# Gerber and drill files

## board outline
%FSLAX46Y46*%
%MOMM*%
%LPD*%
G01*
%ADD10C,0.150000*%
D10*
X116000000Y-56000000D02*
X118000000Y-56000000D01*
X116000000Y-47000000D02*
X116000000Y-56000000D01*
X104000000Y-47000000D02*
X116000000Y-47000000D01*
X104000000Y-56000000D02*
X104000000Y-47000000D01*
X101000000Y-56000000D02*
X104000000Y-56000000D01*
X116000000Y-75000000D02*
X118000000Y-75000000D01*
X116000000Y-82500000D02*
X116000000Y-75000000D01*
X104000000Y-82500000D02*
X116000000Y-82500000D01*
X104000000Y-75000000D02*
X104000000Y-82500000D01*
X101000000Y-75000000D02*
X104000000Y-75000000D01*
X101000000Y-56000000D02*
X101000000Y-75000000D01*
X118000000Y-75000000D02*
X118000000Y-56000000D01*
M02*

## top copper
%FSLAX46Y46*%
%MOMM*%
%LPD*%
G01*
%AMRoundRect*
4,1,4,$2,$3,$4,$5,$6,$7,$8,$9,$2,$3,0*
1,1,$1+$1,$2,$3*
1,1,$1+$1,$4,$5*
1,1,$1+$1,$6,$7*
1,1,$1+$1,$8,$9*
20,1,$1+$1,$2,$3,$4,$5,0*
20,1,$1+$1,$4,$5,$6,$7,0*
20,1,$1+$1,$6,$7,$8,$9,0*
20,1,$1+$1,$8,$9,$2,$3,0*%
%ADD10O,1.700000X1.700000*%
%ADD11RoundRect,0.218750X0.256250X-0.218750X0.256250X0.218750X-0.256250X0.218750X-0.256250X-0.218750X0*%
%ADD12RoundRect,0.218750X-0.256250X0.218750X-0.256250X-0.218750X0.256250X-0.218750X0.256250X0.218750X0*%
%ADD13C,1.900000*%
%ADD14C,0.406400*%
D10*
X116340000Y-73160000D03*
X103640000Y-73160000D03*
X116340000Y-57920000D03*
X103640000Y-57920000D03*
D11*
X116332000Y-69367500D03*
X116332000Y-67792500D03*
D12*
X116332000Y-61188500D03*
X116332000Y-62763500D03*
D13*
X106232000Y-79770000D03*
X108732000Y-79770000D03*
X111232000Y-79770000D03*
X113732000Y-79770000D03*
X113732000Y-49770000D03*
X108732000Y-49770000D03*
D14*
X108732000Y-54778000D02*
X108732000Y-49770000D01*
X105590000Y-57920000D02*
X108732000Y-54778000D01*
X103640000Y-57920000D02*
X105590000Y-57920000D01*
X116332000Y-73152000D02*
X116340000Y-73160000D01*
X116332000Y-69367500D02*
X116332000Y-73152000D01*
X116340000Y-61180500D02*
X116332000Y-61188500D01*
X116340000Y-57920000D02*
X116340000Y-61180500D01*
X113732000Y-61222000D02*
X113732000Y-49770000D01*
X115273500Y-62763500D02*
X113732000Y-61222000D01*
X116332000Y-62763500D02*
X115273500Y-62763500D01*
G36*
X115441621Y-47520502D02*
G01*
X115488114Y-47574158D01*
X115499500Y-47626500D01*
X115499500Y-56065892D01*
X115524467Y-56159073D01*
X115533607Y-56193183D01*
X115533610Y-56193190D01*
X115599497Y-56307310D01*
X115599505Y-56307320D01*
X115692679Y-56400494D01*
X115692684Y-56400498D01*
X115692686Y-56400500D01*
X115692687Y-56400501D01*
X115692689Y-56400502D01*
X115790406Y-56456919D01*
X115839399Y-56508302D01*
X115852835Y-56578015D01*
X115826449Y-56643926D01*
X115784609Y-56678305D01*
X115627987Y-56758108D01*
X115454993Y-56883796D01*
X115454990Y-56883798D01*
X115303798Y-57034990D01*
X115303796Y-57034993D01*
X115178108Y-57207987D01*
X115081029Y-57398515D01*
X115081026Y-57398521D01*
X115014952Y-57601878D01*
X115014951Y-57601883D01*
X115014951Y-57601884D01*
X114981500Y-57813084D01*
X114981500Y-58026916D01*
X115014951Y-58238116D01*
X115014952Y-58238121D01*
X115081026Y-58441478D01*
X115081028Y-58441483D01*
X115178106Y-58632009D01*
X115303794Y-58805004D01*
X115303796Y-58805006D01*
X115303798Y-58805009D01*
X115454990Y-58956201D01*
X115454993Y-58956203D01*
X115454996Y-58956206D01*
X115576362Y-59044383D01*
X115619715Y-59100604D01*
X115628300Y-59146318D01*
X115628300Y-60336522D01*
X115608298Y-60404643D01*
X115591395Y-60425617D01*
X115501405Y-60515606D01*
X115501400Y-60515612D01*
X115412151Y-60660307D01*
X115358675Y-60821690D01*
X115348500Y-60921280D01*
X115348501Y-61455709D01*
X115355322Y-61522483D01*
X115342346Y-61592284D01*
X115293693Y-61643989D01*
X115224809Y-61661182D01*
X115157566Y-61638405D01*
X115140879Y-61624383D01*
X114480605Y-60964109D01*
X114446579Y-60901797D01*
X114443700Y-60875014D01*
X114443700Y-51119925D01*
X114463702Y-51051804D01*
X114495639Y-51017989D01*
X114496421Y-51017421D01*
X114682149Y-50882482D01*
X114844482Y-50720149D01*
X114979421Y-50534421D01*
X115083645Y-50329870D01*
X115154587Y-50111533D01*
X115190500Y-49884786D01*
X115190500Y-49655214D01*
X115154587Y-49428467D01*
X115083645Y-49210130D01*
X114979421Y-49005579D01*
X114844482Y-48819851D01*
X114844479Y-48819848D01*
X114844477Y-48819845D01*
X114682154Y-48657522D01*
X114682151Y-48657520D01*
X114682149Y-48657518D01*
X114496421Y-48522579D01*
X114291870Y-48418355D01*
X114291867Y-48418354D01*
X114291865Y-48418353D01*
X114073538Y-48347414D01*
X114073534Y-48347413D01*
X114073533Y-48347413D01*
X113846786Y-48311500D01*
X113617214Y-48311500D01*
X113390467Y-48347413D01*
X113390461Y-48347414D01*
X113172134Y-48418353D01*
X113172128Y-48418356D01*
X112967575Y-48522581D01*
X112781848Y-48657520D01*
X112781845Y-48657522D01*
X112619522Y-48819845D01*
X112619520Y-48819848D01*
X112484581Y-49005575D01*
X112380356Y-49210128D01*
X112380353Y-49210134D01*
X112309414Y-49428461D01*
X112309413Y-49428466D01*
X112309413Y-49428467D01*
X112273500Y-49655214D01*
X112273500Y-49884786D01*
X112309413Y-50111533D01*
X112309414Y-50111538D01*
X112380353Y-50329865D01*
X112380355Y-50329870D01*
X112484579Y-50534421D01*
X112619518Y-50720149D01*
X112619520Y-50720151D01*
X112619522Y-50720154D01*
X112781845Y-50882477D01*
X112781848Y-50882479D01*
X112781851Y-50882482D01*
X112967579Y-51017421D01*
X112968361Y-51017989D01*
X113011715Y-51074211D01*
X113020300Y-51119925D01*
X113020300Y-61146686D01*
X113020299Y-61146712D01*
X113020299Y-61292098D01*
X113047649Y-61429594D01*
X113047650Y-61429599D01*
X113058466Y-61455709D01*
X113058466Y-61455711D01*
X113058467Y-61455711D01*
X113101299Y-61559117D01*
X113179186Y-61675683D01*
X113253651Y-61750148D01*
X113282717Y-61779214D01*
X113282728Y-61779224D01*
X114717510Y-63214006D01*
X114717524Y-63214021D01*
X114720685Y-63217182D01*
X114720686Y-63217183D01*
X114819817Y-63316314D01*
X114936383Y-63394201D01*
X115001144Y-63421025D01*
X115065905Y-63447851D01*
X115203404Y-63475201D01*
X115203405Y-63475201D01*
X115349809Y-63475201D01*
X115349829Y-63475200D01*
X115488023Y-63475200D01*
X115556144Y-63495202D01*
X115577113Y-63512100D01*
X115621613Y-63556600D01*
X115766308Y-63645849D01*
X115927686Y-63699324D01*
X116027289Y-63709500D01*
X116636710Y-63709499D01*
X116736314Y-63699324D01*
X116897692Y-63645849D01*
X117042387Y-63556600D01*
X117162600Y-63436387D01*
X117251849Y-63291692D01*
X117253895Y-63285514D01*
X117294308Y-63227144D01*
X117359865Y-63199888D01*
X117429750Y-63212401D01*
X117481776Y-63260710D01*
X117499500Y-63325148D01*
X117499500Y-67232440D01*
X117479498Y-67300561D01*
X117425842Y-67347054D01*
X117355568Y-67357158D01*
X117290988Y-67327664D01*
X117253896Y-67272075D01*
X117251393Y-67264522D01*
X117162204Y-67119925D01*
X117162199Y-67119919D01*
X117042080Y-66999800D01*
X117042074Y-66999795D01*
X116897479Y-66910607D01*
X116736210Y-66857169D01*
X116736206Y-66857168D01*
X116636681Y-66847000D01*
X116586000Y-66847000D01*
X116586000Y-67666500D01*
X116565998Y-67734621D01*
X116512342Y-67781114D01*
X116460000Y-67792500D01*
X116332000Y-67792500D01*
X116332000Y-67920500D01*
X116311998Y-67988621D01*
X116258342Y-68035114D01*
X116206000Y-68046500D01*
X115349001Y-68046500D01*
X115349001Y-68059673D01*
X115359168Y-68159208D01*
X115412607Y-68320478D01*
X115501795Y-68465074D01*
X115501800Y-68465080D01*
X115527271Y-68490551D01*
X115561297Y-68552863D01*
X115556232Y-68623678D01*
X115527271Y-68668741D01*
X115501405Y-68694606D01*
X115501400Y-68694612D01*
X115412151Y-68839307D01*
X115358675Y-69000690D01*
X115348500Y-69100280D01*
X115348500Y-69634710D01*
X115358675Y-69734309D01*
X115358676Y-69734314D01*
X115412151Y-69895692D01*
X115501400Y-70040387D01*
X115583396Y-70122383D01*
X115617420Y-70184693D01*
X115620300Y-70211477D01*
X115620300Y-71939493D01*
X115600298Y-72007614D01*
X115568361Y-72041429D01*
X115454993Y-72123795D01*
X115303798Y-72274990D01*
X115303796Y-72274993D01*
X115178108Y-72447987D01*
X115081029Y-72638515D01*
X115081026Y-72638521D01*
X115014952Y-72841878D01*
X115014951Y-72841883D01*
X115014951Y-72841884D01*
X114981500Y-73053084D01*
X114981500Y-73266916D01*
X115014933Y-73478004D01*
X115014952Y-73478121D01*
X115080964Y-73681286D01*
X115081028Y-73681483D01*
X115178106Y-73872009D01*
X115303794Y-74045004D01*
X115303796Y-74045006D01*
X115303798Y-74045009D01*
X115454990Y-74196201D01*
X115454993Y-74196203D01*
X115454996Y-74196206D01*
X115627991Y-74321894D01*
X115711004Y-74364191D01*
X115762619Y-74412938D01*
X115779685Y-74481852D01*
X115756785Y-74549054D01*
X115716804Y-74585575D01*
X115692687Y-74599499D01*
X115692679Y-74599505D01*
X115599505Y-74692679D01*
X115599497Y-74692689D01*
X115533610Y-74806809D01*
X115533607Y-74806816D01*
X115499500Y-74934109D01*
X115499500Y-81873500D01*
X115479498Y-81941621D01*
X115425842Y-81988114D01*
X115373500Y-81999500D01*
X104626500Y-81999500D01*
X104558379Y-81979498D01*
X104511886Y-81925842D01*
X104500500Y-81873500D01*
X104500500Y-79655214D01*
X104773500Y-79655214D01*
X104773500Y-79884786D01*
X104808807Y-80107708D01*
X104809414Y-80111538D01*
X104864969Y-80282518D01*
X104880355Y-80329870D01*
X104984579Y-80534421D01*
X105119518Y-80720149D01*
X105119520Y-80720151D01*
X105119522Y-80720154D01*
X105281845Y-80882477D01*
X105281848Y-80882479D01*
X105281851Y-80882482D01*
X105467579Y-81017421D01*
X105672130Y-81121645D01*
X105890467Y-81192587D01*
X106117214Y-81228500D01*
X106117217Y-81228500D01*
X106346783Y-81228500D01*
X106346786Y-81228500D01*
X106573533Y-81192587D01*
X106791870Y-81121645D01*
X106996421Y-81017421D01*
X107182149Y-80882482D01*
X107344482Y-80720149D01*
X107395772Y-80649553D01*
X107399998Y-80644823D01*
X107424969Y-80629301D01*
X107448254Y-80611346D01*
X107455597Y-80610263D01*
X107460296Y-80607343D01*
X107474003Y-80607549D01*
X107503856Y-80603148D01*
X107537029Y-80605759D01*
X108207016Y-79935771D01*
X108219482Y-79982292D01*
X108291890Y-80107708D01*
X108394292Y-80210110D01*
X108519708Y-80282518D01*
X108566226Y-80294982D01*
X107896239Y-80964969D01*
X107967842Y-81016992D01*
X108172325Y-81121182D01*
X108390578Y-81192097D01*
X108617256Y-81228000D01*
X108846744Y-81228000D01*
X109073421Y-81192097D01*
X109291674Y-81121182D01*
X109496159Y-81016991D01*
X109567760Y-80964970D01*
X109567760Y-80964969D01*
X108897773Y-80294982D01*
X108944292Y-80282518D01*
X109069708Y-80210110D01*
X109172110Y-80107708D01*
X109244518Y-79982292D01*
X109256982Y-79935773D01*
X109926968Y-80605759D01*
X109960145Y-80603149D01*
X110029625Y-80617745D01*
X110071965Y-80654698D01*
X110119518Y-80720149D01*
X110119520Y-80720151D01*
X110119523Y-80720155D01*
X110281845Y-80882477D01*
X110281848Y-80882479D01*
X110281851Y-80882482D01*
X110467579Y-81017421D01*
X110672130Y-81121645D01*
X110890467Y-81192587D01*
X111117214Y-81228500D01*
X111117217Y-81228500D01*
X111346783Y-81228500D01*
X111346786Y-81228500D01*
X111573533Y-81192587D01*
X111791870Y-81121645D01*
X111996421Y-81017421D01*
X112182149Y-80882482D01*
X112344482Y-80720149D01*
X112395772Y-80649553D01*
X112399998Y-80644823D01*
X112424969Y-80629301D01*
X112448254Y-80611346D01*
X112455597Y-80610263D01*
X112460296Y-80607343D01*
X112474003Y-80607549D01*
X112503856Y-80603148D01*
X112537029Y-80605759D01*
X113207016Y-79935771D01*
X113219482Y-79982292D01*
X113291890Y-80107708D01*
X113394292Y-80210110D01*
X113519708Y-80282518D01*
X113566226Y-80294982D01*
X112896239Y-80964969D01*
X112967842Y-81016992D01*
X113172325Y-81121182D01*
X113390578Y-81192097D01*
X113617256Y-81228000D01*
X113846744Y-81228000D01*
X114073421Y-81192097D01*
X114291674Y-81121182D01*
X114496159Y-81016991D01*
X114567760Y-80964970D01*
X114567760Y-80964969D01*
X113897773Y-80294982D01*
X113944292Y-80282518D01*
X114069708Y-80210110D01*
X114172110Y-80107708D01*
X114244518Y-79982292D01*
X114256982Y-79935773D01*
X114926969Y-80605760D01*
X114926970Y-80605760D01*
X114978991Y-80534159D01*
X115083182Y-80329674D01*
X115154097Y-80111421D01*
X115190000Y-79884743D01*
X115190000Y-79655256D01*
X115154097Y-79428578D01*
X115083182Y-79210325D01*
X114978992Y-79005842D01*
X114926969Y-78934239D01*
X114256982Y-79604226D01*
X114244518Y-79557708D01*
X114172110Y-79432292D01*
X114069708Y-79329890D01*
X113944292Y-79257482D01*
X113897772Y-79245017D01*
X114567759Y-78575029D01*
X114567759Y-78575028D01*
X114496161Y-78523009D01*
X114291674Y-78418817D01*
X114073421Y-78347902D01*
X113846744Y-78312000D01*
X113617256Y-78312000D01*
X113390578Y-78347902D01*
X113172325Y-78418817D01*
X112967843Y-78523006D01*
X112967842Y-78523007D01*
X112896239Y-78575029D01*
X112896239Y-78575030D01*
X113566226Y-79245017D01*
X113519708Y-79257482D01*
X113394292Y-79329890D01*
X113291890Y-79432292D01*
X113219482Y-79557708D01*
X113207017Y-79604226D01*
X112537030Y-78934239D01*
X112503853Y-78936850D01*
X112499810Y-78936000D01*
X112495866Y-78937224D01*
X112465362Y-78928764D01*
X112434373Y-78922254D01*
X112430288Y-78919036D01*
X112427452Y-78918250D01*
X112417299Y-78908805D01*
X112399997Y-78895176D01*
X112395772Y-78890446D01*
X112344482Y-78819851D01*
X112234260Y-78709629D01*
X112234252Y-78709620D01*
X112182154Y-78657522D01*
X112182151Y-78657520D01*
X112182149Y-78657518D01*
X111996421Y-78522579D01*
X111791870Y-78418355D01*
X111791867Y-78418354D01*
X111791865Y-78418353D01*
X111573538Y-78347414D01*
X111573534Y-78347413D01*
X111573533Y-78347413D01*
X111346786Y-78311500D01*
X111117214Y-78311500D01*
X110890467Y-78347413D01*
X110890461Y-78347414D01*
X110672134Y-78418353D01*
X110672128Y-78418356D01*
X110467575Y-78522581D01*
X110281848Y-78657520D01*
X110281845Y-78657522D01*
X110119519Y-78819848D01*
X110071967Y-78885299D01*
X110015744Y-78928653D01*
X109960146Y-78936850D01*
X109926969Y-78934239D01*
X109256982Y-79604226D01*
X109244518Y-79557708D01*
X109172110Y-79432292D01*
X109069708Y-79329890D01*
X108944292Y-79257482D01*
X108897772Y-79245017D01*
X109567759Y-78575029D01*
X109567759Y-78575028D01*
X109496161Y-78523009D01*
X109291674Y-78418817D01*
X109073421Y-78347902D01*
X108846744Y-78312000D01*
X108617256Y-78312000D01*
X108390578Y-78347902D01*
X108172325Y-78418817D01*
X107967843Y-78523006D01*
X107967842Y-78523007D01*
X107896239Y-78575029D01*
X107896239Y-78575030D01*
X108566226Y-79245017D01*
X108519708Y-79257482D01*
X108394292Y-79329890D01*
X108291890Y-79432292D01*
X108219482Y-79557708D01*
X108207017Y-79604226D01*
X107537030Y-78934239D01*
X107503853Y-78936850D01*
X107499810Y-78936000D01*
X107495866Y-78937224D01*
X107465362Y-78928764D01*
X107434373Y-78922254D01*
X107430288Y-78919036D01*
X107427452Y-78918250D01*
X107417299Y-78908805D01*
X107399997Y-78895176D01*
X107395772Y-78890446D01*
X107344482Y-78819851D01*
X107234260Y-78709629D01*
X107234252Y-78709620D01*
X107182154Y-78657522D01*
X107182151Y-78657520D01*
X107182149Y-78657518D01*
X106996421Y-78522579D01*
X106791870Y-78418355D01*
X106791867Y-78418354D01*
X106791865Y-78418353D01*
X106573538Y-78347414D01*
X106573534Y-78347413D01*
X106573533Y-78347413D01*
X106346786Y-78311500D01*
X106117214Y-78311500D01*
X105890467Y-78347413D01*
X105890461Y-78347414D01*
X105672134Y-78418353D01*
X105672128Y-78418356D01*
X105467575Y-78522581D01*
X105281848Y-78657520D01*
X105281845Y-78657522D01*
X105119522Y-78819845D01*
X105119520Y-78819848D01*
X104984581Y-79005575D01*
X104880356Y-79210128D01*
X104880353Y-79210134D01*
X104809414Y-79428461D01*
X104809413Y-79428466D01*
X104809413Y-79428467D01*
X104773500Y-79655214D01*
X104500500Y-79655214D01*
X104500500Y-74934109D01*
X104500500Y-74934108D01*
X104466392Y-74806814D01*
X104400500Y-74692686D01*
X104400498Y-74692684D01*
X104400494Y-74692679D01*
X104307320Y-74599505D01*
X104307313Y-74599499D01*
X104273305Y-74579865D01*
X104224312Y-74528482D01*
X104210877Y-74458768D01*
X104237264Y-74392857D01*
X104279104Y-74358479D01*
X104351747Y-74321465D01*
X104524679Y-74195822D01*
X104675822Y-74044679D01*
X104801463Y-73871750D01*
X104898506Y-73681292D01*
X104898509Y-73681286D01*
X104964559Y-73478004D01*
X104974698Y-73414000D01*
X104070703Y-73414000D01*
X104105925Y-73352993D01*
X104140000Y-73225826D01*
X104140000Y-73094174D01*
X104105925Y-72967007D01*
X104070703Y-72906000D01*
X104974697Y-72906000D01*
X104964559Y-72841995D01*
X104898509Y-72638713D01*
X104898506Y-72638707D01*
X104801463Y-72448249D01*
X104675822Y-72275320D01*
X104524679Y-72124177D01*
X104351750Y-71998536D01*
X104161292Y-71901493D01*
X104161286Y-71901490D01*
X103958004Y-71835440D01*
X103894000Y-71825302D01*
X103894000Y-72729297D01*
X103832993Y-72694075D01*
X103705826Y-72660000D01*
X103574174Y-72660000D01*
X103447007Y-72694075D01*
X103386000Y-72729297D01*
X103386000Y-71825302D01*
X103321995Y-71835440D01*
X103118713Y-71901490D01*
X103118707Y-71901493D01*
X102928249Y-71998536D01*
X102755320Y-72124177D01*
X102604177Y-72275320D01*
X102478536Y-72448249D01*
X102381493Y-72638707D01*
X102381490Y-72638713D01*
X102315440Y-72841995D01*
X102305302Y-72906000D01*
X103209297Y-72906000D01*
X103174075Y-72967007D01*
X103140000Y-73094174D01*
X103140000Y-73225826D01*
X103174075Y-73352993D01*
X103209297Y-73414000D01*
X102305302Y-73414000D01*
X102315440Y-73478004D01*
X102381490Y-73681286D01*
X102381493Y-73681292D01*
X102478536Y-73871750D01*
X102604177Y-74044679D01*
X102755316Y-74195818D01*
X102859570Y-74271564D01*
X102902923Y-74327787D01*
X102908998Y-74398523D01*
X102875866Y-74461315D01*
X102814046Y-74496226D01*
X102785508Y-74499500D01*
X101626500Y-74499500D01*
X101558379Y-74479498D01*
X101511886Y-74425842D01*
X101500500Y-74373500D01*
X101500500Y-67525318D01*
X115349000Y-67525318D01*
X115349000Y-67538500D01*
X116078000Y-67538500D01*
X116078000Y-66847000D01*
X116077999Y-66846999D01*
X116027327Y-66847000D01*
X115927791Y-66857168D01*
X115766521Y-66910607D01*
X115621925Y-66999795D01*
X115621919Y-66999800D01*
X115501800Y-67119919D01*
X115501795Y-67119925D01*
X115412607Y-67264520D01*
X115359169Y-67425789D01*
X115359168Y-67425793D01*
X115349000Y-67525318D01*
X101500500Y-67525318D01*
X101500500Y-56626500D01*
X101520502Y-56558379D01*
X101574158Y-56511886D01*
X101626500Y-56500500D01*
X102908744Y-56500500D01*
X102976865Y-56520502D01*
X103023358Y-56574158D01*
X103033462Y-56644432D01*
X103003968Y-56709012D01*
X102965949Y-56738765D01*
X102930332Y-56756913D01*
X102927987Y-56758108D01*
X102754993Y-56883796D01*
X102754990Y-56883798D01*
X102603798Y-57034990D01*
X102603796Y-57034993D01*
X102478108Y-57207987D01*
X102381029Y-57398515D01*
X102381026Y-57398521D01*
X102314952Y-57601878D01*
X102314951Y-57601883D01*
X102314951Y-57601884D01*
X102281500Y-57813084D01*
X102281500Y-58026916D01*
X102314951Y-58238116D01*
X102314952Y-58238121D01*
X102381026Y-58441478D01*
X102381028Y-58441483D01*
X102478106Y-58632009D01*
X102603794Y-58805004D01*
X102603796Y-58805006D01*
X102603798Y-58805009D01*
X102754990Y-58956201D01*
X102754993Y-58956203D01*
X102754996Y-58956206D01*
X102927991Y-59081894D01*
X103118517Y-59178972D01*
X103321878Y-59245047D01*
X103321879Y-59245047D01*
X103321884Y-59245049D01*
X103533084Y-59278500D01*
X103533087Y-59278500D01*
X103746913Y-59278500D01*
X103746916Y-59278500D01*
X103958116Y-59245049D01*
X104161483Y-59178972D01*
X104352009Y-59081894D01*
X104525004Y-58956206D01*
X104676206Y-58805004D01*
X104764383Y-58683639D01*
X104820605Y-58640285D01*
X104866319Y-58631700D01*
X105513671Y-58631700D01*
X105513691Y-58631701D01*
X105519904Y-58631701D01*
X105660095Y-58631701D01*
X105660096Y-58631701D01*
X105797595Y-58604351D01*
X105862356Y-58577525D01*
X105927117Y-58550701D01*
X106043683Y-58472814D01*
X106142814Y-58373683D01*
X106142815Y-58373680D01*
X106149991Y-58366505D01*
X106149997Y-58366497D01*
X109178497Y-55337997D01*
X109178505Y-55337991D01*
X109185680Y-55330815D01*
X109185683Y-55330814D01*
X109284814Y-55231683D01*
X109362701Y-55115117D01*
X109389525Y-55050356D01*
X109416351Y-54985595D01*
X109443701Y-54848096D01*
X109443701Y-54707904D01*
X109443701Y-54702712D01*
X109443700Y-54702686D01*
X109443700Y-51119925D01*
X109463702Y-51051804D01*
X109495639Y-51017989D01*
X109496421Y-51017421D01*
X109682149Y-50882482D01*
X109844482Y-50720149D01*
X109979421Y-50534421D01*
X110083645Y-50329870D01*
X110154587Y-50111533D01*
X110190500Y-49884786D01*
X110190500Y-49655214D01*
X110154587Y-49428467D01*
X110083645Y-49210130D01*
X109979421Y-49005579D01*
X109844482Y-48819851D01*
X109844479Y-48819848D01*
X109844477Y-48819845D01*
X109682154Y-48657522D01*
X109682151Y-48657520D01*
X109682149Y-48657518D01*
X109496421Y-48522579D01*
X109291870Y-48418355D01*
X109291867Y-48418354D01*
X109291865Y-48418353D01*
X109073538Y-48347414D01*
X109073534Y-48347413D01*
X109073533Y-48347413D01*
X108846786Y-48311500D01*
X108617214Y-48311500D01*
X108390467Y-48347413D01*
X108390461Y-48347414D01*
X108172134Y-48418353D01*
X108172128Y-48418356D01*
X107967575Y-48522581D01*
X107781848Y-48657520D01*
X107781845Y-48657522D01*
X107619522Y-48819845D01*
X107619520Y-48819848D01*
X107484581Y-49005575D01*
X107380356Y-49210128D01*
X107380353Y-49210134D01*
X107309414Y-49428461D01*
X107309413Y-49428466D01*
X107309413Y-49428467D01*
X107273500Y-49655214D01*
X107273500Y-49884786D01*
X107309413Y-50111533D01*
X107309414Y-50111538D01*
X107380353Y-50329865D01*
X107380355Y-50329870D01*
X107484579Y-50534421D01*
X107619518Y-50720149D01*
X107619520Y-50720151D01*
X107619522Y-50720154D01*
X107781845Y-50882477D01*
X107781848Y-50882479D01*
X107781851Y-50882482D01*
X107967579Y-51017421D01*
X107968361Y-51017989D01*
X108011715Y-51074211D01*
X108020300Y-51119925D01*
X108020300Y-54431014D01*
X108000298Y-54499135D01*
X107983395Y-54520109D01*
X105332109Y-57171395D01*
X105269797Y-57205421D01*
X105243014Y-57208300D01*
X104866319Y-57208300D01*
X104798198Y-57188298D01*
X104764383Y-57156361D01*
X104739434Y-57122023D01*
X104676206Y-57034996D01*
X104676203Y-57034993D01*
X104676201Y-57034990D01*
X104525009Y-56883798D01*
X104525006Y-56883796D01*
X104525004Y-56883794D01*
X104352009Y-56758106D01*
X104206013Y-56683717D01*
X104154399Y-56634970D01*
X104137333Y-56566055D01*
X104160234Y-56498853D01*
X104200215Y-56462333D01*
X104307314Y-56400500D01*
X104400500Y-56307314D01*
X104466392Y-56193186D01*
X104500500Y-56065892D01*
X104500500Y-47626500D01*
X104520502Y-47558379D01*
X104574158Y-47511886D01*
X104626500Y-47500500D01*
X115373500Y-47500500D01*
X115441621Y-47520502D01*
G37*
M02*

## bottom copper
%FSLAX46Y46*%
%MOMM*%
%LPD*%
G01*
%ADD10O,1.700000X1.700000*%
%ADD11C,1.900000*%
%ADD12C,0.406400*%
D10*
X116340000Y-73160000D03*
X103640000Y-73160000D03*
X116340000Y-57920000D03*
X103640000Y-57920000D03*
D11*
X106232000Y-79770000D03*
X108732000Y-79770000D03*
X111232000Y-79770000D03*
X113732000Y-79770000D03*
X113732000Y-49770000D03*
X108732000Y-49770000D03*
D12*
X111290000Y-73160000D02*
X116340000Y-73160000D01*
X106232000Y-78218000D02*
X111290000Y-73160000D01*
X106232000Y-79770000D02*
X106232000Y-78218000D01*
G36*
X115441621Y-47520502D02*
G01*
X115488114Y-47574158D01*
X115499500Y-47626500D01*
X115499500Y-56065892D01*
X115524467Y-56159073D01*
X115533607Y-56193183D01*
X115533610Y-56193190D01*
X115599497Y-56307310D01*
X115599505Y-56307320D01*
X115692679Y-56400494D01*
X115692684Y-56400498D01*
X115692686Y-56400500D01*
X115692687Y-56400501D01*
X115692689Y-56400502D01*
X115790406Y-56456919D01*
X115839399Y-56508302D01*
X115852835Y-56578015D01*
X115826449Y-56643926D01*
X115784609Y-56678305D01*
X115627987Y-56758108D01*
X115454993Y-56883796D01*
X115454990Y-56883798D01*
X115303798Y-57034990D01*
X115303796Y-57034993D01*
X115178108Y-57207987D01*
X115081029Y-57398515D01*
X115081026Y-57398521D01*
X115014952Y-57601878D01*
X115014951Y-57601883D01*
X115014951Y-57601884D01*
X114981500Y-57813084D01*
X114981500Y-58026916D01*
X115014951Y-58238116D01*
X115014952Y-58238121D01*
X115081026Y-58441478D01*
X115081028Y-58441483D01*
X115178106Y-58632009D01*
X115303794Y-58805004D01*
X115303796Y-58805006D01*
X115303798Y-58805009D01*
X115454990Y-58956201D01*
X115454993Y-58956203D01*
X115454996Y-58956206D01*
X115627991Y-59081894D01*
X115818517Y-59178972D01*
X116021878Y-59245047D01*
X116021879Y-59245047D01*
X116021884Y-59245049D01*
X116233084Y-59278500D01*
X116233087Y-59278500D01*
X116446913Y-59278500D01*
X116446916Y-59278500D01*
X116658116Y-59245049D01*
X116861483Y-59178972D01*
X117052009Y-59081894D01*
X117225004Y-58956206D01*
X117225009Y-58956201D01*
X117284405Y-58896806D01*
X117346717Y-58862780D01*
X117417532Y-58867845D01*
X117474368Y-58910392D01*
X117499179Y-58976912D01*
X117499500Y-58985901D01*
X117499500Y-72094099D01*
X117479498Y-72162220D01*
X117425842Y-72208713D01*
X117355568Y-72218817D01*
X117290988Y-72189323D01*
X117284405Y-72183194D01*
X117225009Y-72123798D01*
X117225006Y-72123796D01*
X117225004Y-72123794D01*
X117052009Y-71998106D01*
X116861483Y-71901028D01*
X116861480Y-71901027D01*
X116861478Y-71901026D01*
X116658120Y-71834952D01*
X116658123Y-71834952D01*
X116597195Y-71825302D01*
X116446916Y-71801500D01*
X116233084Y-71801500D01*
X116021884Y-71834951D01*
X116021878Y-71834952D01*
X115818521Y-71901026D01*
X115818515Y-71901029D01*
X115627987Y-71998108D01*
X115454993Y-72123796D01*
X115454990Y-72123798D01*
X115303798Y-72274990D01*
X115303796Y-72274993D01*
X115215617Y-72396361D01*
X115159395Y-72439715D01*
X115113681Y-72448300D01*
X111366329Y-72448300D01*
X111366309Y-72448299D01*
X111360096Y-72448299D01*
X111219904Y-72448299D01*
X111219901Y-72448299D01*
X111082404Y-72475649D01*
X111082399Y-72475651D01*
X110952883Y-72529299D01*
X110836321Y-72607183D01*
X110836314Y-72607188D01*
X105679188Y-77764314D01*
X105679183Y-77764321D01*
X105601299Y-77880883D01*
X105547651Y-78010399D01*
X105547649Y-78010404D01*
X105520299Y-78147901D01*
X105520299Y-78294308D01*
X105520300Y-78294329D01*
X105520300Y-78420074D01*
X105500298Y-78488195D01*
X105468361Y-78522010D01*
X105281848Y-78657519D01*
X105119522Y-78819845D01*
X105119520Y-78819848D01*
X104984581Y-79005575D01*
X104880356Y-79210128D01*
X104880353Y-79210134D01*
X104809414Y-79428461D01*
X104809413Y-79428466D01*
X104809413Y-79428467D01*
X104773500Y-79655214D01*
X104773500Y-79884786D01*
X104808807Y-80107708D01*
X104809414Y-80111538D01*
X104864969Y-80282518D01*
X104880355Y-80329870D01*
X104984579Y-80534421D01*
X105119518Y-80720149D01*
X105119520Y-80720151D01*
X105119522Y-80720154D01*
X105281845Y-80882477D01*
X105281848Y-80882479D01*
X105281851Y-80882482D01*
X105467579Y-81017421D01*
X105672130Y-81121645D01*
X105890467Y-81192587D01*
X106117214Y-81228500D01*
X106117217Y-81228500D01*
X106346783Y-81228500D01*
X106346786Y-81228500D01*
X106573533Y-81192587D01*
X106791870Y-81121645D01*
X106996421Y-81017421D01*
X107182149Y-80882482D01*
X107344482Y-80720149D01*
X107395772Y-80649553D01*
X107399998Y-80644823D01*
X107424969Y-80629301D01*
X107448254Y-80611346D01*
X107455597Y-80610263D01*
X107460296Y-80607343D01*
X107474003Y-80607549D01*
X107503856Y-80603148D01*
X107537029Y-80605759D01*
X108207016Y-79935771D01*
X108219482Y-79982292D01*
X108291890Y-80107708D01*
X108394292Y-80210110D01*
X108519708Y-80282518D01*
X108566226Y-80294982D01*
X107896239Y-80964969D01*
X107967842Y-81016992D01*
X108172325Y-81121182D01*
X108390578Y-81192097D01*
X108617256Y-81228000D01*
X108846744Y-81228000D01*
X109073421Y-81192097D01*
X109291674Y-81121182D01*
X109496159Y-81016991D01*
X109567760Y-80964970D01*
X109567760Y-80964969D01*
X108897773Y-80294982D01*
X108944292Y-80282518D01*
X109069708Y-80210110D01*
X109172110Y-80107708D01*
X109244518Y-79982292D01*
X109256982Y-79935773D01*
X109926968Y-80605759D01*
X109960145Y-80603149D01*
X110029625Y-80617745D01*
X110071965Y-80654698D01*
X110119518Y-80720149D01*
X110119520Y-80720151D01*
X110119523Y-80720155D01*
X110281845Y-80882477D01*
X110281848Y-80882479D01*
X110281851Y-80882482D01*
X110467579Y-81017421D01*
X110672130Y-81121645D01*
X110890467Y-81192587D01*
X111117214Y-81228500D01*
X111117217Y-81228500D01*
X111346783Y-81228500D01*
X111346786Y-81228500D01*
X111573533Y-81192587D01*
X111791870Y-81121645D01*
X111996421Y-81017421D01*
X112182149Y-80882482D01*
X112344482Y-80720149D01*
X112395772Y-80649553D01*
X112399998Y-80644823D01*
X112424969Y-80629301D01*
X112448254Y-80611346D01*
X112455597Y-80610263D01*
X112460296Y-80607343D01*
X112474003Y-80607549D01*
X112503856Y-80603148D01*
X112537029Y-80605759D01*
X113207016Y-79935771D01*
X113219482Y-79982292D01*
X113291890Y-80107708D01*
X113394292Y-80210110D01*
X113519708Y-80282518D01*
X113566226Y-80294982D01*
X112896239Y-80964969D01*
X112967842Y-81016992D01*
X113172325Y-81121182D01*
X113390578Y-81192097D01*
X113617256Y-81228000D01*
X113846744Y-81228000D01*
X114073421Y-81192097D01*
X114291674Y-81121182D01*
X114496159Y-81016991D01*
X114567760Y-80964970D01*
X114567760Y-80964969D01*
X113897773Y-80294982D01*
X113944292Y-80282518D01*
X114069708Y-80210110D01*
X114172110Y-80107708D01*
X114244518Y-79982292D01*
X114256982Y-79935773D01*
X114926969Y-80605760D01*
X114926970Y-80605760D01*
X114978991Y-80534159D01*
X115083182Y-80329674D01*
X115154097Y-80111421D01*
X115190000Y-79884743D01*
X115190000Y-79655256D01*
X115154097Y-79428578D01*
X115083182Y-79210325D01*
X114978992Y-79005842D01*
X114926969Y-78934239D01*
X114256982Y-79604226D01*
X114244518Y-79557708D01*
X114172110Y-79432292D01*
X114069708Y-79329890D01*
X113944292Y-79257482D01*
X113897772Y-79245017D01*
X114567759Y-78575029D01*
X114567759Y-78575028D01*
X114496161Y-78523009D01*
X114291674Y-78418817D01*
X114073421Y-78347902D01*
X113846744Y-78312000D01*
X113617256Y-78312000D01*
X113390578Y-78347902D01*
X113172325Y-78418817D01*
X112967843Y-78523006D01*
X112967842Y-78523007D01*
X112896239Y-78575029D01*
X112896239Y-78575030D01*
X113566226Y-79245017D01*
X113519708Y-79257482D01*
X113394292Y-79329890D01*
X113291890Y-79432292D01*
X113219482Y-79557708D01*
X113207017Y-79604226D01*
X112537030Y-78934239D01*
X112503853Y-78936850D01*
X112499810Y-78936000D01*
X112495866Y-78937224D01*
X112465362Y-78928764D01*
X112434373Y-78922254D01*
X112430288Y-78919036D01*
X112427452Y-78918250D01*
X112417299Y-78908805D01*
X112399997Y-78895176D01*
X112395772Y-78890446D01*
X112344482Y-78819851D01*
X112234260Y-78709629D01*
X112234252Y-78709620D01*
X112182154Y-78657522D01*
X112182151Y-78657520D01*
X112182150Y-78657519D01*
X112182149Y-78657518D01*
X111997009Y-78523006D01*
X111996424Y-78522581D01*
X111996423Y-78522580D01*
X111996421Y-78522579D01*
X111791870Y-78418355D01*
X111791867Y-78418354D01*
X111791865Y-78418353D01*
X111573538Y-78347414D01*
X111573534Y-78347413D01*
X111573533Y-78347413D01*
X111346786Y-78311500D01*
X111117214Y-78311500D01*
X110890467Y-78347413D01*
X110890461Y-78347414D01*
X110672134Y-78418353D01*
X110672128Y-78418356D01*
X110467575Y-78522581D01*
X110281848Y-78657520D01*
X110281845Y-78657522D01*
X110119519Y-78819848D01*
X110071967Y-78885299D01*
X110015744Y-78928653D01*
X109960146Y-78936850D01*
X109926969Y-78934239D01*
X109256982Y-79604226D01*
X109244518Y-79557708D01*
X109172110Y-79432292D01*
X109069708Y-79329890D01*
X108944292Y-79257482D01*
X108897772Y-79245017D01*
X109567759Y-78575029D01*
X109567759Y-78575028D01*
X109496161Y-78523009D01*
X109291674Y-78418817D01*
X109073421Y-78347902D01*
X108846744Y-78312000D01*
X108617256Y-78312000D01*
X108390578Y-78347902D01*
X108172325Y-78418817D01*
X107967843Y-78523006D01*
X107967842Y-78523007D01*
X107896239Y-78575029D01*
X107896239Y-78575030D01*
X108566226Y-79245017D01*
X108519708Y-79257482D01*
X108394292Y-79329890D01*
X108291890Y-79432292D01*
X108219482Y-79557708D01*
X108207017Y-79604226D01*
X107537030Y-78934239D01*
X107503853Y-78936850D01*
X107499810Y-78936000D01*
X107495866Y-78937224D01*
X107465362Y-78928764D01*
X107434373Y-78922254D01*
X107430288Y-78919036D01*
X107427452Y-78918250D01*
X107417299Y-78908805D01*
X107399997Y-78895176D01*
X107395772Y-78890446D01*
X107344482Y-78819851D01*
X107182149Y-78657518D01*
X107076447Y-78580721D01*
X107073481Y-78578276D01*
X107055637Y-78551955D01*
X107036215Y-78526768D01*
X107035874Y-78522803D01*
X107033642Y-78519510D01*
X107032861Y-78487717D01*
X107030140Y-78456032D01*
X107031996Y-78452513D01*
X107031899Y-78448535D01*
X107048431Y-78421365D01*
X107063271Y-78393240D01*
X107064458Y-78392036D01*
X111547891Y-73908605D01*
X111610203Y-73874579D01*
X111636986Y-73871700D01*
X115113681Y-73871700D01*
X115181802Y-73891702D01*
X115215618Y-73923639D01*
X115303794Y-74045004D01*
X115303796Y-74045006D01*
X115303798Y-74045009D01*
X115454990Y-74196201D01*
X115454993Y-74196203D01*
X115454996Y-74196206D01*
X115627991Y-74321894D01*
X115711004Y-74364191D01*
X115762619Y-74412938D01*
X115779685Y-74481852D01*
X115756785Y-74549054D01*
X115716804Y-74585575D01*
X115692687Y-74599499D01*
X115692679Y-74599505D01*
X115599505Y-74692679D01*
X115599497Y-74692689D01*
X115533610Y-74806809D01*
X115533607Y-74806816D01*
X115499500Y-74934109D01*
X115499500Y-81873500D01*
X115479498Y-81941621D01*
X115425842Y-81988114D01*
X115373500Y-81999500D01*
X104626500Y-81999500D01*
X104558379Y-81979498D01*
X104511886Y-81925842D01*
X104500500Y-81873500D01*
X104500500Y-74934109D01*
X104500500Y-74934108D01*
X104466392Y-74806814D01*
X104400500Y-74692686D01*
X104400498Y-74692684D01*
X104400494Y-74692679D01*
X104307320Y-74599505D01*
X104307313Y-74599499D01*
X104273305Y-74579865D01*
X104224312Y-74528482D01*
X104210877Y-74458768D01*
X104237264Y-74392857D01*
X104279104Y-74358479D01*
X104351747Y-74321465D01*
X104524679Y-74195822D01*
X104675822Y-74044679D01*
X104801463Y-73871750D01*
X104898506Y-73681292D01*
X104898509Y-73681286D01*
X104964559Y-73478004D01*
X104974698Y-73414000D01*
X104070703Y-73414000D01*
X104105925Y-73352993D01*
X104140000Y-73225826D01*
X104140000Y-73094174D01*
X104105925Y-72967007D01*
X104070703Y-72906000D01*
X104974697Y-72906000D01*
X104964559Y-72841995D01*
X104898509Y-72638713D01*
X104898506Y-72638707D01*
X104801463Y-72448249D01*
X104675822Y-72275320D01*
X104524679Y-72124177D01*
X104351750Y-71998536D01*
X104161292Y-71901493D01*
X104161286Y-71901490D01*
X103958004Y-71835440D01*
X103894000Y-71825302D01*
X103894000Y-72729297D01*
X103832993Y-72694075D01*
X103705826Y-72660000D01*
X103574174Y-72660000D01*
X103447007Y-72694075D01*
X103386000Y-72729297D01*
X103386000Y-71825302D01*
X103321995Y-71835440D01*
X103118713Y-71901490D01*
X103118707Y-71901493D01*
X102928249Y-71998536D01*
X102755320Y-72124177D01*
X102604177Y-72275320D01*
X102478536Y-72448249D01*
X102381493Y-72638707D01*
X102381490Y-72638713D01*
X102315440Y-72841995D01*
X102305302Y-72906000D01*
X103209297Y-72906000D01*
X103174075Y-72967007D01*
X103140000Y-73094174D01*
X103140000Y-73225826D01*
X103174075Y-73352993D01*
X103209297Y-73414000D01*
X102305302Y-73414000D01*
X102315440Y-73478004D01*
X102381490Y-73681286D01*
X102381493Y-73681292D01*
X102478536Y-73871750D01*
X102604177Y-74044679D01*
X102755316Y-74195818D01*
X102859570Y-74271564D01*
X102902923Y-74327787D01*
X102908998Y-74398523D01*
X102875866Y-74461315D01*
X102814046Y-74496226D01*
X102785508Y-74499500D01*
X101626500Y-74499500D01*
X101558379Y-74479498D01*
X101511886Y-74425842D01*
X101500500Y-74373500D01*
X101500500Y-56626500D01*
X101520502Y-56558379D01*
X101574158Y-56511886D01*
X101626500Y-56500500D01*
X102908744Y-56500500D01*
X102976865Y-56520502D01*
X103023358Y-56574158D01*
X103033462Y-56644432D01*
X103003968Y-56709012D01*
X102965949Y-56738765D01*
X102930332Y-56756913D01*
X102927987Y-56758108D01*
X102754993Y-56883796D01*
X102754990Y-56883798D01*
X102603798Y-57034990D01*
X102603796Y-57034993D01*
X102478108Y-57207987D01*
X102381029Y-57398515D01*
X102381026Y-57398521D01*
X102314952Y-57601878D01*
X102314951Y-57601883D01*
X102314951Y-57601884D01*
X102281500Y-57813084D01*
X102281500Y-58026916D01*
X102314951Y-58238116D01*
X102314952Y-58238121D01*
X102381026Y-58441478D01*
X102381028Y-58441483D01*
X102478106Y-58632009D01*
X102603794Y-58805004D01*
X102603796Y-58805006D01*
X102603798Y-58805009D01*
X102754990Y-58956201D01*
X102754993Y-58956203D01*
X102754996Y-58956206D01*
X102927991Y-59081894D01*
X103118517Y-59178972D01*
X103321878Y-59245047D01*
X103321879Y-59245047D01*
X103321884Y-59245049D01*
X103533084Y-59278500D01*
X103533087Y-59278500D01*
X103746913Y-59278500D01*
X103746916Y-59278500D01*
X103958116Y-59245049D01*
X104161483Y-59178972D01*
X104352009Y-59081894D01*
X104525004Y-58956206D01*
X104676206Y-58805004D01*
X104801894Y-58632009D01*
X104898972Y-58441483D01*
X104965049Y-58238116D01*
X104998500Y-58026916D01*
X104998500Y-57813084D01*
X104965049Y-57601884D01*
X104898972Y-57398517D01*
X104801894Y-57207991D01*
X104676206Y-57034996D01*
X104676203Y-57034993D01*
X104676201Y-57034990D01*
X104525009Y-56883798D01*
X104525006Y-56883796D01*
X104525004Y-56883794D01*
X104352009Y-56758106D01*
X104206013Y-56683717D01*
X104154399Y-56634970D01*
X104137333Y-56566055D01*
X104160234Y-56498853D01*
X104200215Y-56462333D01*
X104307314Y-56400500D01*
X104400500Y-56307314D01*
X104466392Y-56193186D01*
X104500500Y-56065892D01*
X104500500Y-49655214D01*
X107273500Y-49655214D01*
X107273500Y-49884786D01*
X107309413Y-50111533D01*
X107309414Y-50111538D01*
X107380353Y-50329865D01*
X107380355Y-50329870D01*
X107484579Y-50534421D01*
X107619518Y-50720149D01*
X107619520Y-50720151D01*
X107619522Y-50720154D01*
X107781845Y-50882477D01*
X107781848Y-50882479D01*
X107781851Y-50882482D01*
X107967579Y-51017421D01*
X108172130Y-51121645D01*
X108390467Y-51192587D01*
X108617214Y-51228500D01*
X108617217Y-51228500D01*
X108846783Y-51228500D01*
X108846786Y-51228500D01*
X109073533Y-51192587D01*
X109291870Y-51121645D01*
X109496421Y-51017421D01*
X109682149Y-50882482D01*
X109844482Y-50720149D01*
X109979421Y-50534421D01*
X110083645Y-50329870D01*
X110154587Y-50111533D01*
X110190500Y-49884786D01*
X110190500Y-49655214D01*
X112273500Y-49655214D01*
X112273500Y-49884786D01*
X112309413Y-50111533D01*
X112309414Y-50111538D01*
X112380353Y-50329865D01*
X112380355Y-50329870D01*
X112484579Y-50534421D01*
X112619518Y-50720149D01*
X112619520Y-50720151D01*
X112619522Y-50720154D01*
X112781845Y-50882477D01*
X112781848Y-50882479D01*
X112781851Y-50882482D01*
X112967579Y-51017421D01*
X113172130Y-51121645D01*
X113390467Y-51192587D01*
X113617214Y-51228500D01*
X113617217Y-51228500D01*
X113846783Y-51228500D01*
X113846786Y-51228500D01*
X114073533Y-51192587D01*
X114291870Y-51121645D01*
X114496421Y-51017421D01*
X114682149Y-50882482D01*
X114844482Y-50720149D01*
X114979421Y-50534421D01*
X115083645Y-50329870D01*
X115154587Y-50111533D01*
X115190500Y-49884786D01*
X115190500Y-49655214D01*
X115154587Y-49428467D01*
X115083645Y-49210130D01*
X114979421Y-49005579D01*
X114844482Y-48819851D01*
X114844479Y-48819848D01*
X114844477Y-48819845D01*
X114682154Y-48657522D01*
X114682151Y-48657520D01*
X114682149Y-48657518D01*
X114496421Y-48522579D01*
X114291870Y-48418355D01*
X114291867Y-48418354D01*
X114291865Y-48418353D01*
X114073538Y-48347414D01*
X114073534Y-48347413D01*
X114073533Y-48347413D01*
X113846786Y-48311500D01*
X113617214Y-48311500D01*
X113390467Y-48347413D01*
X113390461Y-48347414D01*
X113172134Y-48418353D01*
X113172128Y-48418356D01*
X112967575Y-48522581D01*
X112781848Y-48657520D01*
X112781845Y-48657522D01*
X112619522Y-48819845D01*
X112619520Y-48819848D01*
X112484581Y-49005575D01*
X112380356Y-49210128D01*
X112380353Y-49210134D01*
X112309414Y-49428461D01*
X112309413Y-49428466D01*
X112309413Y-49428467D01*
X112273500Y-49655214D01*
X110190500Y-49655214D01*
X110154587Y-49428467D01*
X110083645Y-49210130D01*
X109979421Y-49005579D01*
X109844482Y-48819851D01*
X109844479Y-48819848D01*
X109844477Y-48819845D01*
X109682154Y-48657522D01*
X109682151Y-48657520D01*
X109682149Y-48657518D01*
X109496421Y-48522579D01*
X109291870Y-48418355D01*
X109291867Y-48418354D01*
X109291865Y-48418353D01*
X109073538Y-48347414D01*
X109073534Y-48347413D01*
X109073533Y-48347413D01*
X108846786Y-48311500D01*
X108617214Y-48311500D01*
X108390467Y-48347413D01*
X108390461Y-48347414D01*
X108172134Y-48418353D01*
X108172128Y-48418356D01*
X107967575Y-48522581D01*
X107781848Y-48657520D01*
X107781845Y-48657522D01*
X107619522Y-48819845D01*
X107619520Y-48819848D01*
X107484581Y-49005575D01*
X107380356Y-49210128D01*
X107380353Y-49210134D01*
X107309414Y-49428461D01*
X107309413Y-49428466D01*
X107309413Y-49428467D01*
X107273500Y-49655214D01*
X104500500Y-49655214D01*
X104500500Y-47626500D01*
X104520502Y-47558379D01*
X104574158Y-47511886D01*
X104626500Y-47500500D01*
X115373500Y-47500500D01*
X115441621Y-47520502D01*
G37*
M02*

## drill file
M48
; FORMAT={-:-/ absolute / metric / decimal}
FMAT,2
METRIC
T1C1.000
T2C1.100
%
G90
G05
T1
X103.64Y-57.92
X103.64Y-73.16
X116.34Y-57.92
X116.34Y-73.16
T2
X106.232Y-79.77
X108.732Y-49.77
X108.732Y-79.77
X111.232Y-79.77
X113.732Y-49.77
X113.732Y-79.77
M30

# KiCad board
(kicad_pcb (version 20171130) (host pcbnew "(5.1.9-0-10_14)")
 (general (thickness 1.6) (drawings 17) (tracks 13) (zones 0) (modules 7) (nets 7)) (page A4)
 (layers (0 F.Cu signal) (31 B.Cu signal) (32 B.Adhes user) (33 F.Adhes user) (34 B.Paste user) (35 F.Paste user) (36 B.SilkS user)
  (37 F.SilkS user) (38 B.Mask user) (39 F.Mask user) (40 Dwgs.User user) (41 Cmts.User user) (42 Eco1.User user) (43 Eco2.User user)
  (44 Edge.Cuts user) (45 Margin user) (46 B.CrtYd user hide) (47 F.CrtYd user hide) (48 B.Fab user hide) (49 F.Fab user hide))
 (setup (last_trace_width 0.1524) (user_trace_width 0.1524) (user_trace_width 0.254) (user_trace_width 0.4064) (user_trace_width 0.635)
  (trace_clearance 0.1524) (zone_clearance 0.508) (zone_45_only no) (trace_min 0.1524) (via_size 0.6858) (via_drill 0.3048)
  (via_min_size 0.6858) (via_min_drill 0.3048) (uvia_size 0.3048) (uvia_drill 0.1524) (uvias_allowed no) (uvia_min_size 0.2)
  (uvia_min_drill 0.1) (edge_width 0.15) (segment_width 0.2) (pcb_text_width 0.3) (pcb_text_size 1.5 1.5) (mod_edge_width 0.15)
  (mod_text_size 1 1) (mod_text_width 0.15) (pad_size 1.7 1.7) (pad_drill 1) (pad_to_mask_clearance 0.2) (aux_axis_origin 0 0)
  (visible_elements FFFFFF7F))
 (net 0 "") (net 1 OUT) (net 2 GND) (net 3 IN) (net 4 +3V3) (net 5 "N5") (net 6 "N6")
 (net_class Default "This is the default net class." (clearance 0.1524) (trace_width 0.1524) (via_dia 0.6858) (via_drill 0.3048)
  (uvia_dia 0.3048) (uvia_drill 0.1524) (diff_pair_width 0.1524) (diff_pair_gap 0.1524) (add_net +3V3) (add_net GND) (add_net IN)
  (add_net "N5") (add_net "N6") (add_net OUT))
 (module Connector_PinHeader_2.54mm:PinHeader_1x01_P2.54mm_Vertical (layer B.Cu) (at 116.34 73.16 90)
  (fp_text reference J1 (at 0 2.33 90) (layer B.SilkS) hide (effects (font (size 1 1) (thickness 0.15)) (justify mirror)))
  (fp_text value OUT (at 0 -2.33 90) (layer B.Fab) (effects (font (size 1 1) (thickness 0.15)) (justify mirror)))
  (pad 1 thru_hole oval (at 0 0 90) (size 1.7 1.7) (drill 1) (layers *.Cu *.Mask) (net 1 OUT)))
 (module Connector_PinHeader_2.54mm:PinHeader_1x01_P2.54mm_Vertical (layer B.Cu) (at 103.64 73.16)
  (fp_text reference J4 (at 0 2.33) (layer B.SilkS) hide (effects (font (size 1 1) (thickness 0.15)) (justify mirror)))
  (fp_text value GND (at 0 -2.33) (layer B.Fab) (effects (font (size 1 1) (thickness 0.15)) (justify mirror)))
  (pad 1 thru_hole oval (at 0 0) (size 1.7 1.7) (drill 1) (layers *.Cu *.Mask) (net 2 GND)))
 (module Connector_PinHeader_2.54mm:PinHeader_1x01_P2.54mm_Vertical (layer B.Cu) (at 116.34 57.92 90)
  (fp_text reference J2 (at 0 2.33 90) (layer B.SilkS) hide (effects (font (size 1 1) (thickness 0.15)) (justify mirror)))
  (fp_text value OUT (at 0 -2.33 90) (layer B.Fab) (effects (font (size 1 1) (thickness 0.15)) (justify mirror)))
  (pad 1 thru_hole oval (at 0 0 90) (size 1.7 1.7) (drill 1) (layers *.Cu *.Mask) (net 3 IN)))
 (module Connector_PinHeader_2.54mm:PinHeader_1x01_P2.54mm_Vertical (layer B.Cu) (at 103.64 57.92 270)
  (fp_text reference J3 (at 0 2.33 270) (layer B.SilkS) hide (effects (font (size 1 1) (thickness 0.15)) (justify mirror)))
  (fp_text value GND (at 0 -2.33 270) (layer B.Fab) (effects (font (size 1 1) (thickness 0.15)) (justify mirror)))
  (pad 1 thru_hole oval (at 0 0 270) (size 1.7 1.7) (drill 1) (layers *.Cu *.Mask) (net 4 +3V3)))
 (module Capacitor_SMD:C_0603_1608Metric (layer F.Cu) (at 116.332 68.58 90)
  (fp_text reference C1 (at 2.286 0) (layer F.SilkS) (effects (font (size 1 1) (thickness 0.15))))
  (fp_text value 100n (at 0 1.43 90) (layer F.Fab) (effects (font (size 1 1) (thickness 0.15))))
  (pad 1 smd roundrect (at -0.7875 0 90) (size 0.875 0.95) (layers F.Cu F.Paste F.Mask) (roundrect_rratio 0.25) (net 1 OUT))
  (pad 2 smd roundrect (at 0.7875 0 90) (size 0.875 0.95) (layers F.Cu F.Paste F.Mask) (roundrect_rratio 0.25) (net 2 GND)))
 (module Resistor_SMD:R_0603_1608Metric (layer F.Cu) (at 116.332 61.976 270)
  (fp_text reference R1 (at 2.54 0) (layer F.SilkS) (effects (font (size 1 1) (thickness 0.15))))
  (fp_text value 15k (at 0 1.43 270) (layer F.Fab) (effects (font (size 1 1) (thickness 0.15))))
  (pad 1 smd roundrect (at -0.7875 0 270) (size 0.875 0.95) (layers F.Cu F.Paste F.Mask) (roundrect_rratio 0.25) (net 3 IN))
  (pad 2 smd roundrect (at 0.7875 0 270) (size 0.875 0.95) (layers F.Cu F.Paste F.Mask) (roundrect_rratio 0.25) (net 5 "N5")))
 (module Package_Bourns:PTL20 (layer F.Cu) (at 109.982 64.77 90)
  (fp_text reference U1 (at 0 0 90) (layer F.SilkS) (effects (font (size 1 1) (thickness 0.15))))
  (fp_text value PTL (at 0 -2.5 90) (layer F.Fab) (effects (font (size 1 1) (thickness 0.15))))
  (pad 1 thru_hole circle (at -15 -3.75 90) (size 1.9 1.9) (drill 1.1) (layers *.Cu *.Mask) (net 1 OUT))
  (pad 2 thru_hole circle (at -15 -1.25 90) (size 1.9 1.9) (drill 1.1) (layers *.Cu *.Mask) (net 2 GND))
  (pad 3 thru_hole circle (at -15 1.25 90) (size 1.9 1.9) (drill 1.1) (layers *.Cu *.Mask) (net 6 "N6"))
  (pad 4 thru_hole circle (at -15 3.75 90) (size 1.9 1.9) (drill 1.1) (layers *.Cu *.Mask) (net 2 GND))
  (pad 5 thru_hole circle (at 15 3.75 90) (size 1.9 1.9) (drill 1.1) (layers *.Cu *.Mask) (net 5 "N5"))
  (pad 6 thru_hole circle (at 15 -1.25 90) (size 1.9 1.9) (drill 1.1) (layers *.Cu *.Mask) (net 4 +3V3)))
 (gr_line (start 116 56) (end 118 56) (layer Edge.Cuts) (width 0.15))
 (gr_line (start 116 47) (end 116 56) (layer Edge.Cuts) (width 0.15))
 (gr_line (start 104 47) (end 116 47) (layer Edge.Cuts) (width 0.15))
 (gr_line (start 104 56) (end 104 47) (layer Edge.Cuts) (width 0.15))
 (gr_line (start 101 56) (end 104 56) (layer Edge.Cuts) (width 0.15))
 (gr_line (start 116 75) (end 118 75) (layer Edge.Cuts) (width 0.15))
 (gr_line (start 116 82.5) (end 116 75) (layer Edge.Cuts) (width 0.15))
 (gr_line (start 104 82.5) (end 116 82.5) (layer Edge.Cuts) (width 0.15))
 (gr_line (start 104 75) (end 104 82.5) (layer Edge.Cuts) (width 0.15))
 (gr_line (start 101 75) (end 104 75) (layer Edge.Cuts) (width 0.15))
 (gr_line (start 101 56) (end 101 75) (layer Edge.Cuts) (width 0.15))
 (gr_line (start 118 75) (end 118 56) (layer Edge.Cuts) (width 0.15))
 (segment (start 108.732 54.778) (end 108.732 49.77) (width 0.4064) (layer F.Cu) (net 4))
 (segment (start 105.59 57.92) (end 108.732 54.778) (width 0.4064) (layer F.Cu) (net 4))
 (segment (start 103.64 57.92) (end 105.59 57.92) (width 0.4064) (layer F.Cu) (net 4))
 (segment (start 111.29 73.16) (end 116.34 73.16) (width 0.4064) (layer B.Cu) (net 1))
 (segment (start 106.232 78.218) (end 111.29 73.16) (width 0.4064) (layer B.Cu) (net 1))
 (segment (start 106.232 79.77) (end 106.232 78.218) (width 0.4064) (layer B.Cu) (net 1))
 (segment (start 116.332 73.152) (end 116.34 73.16) (width 0.4064) (layer F.Cu) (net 1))
 (segment (start 116.332 69.3675) (end 116.332 73.152) (width 0.4064) (layer F.Cu) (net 1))
 (segment (start 116.34 61.1805) (end 116.332 61.1885) (width 0.4064) (layer F.Cu) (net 3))
 (segment (start 116.34 57.92) (end 116.34 61.1805) (width 0.4064) (layer F.Cu) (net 3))
 (segment (start 113.732 61.222) (end 113.732 49.77) (width 0.4064) (layer F.Cu) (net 5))
 (segment (start 115.2735 62.7635) (end 113.732 61.222) (width 0.4064) (layer F.Cu) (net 5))
 (segment (start 116.332 62.7635) (end 115.2735 62.7635) (width 0.4064) (layer F.Cu) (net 5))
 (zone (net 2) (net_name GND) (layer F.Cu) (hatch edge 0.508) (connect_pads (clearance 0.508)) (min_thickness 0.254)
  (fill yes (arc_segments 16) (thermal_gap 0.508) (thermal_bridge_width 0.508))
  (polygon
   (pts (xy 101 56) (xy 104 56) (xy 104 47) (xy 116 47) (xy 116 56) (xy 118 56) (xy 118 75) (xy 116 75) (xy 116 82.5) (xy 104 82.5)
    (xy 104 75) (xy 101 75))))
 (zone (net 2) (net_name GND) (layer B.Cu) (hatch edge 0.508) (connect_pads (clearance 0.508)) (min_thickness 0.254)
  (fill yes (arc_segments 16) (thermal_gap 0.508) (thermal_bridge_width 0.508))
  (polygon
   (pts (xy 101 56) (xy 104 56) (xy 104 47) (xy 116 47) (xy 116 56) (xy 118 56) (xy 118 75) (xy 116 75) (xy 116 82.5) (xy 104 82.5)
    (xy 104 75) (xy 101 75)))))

